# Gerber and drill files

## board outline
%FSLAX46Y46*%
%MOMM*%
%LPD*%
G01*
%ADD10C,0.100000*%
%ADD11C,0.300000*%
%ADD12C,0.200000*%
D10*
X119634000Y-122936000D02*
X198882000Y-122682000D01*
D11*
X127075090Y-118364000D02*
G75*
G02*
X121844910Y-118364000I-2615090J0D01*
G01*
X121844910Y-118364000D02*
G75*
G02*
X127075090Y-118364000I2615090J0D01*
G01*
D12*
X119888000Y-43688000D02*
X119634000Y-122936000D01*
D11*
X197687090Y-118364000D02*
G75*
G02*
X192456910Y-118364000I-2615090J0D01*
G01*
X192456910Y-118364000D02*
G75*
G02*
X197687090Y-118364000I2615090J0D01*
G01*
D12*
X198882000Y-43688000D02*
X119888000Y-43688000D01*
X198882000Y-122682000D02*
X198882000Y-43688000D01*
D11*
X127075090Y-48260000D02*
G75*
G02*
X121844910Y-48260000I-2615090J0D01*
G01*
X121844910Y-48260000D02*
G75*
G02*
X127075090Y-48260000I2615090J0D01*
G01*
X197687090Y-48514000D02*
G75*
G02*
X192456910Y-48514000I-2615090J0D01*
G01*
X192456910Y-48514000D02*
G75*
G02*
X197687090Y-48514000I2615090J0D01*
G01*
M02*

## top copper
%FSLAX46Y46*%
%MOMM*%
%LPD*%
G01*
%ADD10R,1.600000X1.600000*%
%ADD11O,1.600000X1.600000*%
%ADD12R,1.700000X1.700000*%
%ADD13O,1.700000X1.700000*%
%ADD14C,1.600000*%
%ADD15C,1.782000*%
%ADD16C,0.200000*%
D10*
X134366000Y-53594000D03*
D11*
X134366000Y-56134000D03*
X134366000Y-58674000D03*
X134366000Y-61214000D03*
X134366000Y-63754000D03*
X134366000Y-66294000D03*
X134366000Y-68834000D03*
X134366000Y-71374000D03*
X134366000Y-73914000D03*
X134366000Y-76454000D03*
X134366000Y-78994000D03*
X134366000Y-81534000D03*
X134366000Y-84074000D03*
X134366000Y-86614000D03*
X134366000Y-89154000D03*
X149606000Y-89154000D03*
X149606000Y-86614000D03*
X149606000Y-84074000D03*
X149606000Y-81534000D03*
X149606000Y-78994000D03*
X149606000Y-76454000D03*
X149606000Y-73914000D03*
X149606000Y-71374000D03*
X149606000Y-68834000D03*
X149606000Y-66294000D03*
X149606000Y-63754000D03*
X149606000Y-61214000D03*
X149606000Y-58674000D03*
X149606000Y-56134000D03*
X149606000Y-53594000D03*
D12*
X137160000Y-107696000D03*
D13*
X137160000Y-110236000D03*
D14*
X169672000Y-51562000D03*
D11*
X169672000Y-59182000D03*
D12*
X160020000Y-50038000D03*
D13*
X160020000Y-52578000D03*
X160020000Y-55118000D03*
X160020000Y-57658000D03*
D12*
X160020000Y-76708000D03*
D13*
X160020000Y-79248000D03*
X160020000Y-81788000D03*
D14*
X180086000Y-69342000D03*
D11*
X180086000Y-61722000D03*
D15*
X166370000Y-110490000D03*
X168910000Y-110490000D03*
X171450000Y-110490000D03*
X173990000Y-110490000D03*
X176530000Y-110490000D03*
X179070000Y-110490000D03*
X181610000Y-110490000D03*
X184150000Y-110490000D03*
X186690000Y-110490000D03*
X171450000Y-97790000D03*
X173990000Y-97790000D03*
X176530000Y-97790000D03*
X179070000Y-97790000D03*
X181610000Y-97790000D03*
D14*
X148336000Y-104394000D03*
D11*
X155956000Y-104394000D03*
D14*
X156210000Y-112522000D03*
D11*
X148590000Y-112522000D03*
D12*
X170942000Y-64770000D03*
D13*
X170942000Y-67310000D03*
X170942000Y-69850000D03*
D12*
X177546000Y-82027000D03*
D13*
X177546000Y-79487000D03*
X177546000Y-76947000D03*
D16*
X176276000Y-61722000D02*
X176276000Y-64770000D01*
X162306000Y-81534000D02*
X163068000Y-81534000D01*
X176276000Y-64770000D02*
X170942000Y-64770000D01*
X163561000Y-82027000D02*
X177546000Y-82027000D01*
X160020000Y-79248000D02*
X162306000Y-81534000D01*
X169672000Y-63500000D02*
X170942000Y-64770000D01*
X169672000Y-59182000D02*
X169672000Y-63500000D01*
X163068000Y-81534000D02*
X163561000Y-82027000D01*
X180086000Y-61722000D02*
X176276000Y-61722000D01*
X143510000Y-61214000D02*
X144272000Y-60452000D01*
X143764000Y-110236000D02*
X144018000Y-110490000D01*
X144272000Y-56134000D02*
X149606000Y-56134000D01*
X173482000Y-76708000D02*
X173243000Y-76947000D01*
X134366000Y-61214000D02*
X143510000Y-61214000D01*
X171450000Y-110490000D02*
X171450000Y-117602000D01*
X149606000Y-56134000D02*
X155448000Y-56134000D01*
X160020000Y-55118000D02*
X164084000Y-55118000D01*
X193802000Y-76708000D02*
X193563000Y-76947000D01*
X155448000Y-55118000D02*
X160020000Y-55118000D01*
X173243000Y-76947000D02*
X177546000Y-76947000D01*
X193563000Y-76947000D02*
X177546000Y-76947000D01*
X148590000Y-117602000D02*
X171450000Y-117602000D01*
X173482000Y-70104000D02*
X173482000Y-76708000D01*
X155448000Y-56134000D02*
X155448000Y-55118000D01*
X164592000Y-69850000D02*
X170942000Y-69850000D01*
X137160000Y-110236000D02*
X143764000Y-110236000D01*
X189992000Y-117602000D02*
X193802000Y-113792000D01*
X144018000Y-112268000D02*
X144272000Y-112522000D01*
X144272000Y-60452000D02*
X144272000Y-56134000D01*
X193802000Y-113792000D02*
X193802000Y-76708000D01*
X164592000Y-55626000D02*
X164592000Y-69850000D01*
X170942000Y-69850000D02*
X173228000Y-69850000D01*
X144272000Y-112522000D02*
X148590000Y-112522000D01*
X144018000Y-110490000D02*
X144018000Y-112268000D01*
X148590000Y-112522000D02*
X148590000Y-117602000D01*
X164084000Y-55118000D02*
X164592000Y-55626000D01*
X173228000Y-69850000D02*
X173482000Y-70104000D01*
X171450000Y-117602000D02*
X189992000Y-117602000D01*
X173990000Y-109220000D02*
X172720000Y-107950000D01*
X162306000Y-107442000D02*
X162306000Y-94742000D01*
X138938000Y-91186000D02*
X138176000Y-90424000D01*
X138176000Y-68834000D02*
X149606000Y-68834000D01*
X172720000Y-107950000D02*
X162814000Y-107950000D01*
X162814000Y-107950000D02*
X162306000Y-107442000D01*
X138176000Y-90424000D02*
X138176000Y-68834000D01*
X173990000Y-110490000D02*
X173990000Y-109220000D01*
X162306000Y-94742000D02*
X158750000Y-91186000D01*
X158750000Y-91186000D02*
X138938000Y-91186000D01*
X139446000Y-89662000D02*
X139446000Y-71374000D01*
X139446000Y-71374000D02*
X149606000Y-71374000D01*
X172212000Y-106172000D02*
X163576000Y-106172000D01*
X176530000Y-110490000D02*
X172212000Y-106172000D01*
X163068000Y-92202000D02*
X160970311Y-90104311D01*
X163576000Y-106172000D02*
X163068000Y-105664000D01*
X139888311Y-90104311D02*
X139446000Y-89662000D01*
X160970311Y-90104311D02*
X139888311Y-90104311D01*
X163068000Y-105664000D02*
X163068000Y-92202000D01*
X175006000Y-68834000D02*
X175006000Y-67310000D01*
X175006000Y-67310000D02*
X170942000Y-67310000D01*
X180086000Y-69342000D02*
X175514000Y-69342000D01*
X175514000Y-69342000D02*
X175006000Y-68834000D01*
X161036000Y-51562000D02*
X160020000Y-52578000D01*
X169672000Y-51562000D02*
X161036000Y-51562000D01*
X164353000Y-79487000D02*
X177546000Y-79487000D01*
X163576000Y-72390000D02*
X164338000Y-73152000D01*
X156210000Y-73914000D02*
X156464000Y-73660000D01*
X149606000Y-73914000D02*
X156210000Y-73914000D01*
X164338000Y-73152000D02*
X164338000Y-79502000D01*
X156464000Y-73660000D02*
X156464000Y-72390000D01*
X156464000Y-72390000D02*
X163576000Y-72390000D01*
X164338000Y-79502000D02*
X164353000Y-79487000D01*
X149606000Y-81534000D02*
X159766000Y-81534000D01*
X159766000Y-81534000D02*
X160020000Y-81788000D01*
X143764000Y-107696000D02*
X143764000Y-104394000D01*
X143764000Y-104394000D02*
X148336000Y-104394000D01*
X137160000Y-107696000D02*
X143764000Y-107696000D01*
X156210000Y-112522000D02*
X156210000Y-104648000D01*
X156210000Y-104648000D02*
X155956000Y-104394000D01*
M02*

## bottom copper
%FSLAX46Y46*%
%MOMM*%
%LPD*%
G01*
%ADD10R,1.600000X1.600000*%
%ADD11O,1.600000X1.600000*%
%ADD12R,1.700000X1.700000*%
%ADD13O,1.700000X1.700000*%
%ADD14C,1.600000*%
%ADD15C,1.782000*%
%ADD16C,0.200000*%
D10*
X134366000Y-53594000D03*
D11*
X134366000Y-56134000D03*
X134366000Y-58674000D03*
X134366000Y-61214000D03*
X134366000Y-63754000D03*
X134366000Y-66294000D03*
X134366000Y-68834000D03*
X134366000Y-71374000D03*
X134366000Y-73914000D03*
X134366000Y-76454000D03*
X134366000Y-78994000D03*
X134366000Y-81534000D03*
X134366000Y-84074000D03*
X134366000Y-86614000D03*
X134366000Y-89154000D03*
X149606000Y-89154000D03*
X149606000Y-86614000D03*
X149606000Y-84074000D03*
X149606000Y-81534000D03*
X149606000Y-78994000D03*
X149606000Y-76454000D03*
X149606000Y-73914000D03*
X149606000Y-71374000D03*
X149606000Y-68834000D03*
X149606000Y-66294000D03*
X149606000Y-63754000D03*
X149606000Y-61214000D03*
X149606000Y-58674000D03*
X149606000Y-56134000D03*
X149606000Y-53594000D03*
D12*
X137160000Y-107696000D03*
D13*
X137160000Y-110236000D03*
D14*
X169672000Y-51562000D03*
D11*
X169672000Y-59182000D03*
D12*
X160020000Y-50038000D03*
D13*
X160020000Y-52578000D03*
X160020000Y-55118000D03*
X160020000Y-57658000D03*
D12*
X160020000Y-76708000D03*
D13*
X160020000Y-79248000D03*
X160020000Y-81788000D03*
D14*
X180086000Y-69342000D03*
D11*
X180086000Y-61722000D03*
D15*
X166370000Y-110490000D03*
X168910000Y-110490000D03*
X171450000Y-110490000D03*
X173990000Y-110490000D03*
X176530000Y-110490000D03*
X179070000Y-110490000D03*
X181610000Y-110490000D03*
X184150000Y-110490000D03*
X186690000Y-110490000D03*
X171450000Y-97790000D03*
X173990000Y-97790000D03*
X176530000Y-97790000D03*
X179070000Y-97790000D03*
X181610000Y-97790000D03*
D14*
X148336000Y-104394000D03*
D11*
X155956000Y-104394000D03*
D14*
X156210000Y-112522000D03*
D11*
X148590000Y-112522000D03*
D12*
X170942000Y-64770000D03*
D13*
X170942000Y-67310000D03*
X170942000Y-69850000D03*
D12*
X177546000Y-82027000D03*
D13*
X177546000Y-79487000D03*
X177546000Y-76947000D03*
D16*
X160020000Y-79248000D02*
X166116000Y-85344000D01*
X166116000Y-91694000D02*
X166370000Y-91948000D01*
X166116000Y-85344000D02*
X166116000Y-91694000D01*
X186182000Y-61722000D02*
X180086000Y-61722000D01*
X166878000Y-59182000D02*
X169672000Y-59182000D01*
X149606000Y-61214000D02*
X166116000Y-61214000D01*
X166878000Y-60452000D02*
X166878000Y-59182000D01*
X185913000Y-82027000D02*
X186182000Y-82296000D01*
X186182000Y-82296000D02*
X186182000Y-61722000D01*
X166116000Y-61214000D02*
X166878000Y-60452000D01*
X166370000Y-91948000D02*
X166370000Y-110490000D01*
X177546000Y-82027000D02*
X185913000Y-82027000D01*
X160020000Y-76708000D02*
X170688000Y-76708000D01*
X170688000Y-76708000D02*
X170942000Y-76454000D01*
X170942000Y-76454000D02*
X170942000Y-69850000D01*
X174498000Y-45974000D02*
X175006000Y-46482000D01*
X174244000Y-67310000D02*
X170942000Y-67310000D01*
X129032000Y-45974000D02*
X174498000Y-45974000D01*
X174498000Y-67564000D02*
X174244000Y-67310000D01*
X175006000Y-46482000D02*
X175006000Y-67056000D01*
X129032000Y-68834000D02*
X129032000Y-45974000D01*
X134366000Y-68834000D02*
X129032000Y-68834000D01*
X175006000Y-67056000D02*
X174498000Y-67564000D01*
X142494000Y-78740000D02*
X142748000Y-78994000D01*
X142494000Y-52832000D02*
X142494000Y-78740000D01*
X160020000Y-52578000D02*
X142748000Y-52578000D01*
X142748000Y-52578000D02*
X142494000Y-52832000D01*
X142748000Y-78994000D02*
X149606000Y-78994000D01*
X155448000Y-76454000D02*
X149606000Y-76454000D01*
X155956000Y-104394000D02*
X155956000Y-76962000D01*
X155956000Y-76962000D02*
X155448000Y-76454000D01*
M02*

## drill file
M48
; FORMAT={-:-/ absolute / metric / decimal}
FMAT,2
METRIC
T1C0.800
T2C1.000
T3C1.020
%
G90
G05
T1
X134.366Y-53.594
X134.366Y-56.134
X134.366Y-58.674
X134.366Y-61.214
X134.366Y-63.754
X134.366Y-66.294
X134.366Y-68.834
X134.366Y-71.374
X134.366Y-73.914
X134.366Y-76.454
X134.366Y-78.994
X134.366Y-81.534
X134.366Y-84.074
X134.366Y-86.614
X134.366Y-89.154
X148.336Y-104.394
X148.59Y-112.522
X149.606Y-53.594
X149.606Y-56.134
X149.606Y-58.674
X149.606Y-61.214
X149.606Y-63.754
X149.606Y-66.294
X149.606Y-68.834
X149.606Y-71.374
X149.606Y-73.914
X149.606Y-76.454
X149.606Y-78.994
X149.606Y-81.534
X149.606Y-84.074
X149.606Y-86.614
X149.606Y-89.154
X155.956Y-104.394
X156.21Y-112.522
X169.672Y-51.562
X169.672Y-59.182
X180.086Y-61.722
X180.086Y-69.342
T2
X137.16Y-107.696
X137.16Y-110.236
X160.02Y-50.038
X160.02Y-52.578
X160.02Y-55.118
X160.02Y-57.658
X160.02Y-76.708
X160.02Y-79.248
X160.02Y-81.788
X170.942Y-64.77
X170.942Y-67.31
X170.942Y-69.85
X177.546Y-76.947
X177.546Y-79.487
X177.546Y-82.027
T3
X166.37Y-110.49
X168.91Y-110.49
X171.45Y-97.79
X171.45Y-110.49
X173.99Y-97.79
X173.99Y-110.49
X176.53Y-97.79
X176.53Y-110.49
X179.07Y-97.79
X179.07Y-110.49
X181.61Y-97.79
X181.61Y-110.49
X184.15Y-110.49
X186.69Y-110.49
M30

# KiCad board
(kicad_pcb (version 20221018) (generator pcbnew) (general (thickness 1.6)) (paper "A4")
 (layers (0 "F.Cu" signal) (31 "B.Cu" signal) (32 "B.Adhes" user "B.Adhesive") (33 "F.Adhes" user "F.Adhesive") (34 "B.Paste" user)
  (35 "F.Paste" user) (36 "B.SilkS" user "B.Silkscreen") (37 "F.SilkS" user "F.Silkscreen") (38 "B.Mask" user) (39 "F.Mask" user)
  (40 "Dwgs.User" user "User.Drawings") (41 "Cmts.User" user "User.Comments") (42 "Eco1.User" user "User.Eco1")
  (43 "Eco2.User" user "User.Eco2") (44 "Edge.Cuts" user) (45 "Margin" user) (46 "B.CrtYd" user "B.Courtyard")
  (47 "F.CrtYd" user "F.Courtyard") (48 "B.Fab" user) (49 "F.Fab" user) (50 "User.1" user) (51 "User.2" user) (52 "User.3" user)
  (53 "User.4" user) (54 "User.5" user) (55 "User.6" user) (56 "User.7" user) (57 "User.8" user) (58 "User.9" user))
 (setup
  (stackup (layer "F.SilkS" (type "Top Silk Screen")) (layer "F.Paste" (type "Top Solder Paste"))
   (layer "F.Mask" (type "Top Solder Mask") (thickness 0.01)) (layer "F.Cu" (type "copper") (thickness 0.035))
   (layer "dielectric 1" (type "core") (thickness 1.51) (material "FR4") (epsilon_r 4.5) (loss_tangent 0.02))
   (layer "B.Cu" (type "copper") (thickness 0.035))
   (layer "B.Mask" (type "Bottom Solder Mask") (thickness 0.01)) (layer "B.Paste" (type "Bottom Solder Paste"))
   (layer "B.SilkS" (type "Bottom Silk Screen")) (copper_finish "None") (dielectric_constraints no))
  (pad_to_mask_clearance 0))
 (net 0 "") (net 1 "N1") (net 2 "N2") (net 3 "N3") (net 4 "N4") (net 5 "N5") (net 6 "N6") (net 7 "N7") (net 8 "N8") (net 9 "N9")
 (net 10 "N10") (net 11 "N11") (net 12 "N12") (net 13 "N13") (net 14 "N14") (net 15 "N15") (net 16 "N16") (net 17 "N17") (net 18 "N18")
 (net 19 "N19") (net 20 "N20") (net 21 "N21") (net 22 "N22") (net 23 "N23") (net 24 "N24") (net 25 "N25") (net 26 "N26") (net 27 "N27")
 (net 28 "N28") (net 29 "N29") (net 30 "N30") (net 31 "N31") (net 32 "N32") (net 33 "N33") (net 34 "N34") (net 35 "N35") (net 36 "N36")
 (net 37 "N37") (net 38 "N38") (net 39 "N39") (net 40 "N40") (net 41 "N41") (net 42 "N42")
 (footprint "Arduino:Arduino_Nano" (layer "F.Cu") (at 134.366 53.594)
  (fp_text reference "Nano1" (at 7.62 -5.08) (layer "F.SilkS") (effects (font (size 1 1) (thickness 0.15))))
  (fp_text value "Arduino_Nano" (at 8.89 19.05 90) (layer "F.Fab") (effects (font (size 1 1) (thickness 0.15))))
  (pad "1" thru_hole rect (at 0 0) (size 1.6 1.6) (drill 0.8) (layers "*.Cu" "*.Mask") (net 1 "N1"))
  (pad "2" thru_hole oval (at 0 2.54) (size 1.6 1.6) (drill 0.8) (layers "*.Cu" "*.Mask") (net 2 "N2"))
  (pad "3" thru_hole oval (at 0 5.08) (size 1.6 1.6) (drill 0.8) (layers "*.Cu" "*.Mask") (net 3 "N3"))
  (pad "4" thru_hole oval (at 0 7.62) (size 1.6 1.6) (drill 0.8) (layers "*.Cu" "*.Mask") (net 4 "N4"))
  (pad "5" thru_hole oval (at 0 10.16) (size 1.6 1.6) (drill 0.8) (layers "*.Cu" "*.Mask") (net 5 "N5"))
  (pad "6" thru_hole oval (at 0 12.7) (size 1.6 1.6) (drill 0.8) (layers "*.Cu" "*.Mask") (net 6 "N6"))
  (pad "7" thru_hole oval (at 0 15.24) (size 1.6 1.6) (drill 0.8) (layers "*.Cu" "*.Mask") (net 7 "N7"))
  (pad "8" thru_hole oval (at 0 17.78) (size 1.6 1.6) (drill 0.8) (layers "*.Cu" "*.Mask") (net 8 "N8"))
  (pad "9" thru_hole oval (at 0 20.32) (size 1.6 1.6) (drill 0.8) (layers "*.Cu" "*.Mask") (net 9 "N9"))
  (pad "10" thru_hole oval (at 0 22.86) (size 1.6 1.6) (drill 0.8) (layers "*.Cu" "*.Mask") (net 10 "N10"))
  (pad "11" thru_hole oval (at 0 25.4) (size 1.6 1.6) (drill 0.8) (layers "*.Cu" "*.Mask") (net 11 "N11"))
  (pad "12" thru_hole oval (at 0 27.94) (size 1.6 1.6) (drill 0.8) (layers "*.Cu" "*.Mask") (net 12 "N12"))
  (pad "13" thru_hole oval (at 0 30.48) (size 1.6 1.6) (drill 0.8) (layers "*.Cu" "*.Mask") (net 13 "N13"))
  (pad "14" thru_hole oval (at 0 33.02) (size 1.6 1.6) (drill 0.8) (layers "*.Cu" "*.Mask") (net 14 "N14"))
  (pad "15" thru_hole oval (at 0 35.56) (size 1.6 1.6) (drill 0.8) (layers "*.Cu" "*.Mask") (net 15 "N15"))
  (pad "16" thru_hole oval (at 15.24 35.56) (size 1.6 1.6) (drill 0.8) (layers "*.Cu" "*.Mask") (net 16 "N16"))
  (pad "17" thru_hole oval (at 15.24 33.02) (size 1.6 1.6) (drill 0.8) (layers "*.Cu" "*.Mask") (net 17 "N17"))
  (pad "18" thru_hole oval (at 15.24 30.48) (size 1.6 1.6) (drill 0.8) (layers "*.Cu" "*.Mask") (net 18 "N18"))
  (pad "19" thru_hole oval (at 15.24 27.94) (size 1.6 1.6) (drill 0.8) (layers "*.Cu" "*.Mask") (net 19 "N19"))
  (pad "20" thru_hole oval (at 15.24 25.4) (size 1.6 1.6) (drill 0.8) (layers "*.Cu" "*.Mask") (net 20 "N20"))
  (pad "21" thru_hole oval (at 15.24 22.86) (size 1.6 1.6) (drill 0.8) (layers "*.Cu" "*.Mask") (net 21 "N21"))
  (pad "22" thru_hole oval (at 15.24 20.32) (size 1.6 1.6) (drill 0.8) (layers "*.Cu" "*.Mask") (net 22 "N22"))
  (pad "23" thru_hole oval (at 15.24 17.78) (size 1.6 1.6) (drill 0.8) (layers "*.Cu" "*.Mask") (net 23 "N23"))
  (pad "24" thru_hole oval (at 15.24 15.24) (size 1.6 1.6) (drill 0.8) (layers "*.Cu" "*.Mask") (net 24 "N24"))
  (pad "25" thru_hole oval (at 15.24 12.7) (size 1.6 1.6) (drill 0.8) (layers "*.Cu" "*.Mask") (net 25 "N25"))
  (pad "26" thru_hole oval (at 15.24 10.16) (size 1.6 1.6) (drill 0.8) (layers "*.Cu" "*.Mask") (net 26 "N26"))
  (pad "27" thru_hole oval (at 15.24 7.62) (size 1.6 1.6) (drill 0.8) (layers "*.Cu" "*.Mask") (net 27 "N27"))
  (pad "28" thru_hole oval (at 15.24 5.08) (size 1.6 1.6) (drill 0.8) (layers "*.Cu" "*.Mask") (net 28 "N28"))
  (pad "29" thru_hole oval (at 15.24 2.54) (size 1.6 1.6) (drill 0.8) (layers "*.Cu" "*.Mask") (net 4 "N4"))
  (pad "30" thru_hole oval (at 15.24 0) (size 1.6 1.6) (drill 0.8) (layers "*.Cu" "*.Mask") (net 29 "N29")))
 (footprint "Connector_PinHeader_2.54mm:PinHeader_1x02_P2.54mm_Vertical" (layer "F.Cu") (at 137.16 107.696)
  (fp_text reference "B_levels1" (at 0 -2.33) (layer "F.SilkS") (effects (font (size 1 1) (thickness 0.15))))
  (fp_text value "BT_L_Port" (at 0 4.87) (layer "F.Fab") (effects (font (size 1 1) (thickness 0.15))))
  (pad "1" thru_hole rect (at 0 0) (size 1.7 1.7) (drill 1) (layers "*.Cu" "*.Mask") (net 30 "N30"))
  (pad "2" thru_hole oval (at 0 2.54) (size 1.7 1.7) (drill 1) (layers "*.Cu" "*.Mask") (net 4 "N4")))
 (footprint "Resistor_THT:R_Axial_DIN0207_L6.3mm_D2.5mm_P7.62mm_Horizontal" (layer "F.Cu") (at 169.672 51.562 -90)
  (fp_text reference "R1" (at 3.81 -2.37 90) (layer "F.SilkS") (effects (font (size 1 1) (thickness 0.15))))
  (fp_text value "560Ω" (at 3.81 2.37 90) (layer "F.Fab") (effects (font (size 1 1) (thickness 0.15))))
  (pad "1" thru_hole circle (at 0 0 270) (size 1.6 1.6) (drill 0.8) (layers "*.Cu" "*.Mask") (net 20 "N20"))
  (pad "2" thru_hole oval (at 7.62 0 270) (size 1.6 1.6) (drill 0.8) (layers "*.Cu" "*.Mask") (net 27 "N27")))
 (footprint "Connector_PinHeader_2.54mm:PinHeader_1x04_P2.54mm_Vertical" (layer "F.Cu") (at 160.02 50.038)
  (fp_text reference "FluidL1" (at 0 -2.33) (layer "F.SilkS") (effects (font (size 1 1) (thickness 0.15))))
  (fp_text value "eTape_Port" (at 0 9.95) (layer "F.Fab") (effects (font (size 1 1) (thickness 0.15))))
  (pad "1" thru_hole rect (at 0 0) (size 1.7 1.7) (drill 1) (layers "*.Cu" "*.Mask") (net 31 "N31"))
  (pad "2" thru_hole oval (at 0 2.54) (size 1.7 1.7) (drill 1) (layers "*.Cu" "*.Mask") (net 20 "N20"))
  (pad "3" thru_hole oval (at 0 5.08) (size 1.7 1.7) (drill 1) (layers "*.Cu" "*.Mask") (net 4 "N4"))
  (pad "4" thru_hole oval (at 0 7.62) (size 1.7 1.7) (drill 1) (layers "*.Cu" "*.Mask") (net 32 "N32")))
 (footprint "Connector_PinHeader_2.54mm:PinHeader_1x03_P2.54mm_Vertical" (layer "F.Cu") (at 160.02 76.708)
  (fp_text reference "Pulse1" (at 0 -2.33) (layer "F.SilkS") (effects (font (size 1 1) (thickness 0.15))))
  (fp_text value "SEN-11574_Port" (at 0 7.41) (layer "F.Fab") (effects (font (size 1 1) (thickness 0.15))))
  (pad "1" thru_hole rect (at 0 0) (size 1.7 1.7) (drill 1) (layers "*.Cu" "*.Mask") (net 4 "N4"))
  (pad "2" thru_hole oval (at 0 2.54) (size 1.7 1.7) (drill 1) (layers "*.Cu" "*.Mask") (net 27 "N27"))
  (pad "3" thru_hole oval (at 0 5.08) (size 1.7 1.7) (drill 1) (layers "*.Cu" "*.Mask") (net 19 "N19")))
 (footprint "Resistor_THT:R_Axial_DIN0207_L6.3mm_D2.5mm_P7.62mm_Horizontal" (layer "F.Cu") (at 180.086 69.342 90)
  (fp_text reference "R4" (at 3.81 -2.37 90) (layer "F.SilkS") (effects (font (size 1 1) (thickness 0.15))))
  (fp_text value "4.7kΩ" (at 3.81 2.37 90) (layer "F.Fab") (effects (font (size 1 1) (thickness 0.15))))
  (pad "1" thru_hole circle (at 0 0 90) (size 1.6 1.6) (drill 0.8) (layers "*.Cu" "*.Mask") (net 7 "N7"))
  (pad "2" thru_hole oval (at 7.62 0 90) (size 1.6 1.6) (drill 0.8) (layers "*.Cu" "*.Mask") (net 27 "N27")))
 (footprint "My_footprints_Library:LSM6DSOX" (layer "F.Cu") (at 176.53 104.14)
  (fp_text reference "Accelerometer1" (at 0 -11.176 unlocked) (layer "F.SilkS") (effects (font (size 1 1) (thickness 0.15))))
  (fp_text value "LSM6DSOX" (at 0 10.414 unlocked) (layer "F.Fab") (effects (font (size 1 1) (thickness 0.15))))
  (pad "1" thru_hole circle (at -10.16 6.35) (size 1.782 1.782) (drill 1.02) (layers "*.Cu" "*.Mask") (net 27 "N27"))
  (pad "2" thru_hole circle (at -7.62 6.35) (size 1.782 1.782) (drill 1.02) (layers "*.Cu" "*.Mask") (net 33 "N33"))
  (pad "3" thru_hole circle (at -5.08 6.35) (size 1.782 1.782) (drill 1.02) (layers "*.Cu" "*.Mask") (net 4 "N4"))
  (pad "4" thru_hole circle (at -2.54 6.35) (size 1.782 1.782) (drill 1.02) (layers "*.Cu" "*.Mask") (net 24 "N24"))
  (pad "5" thru_hole circle (at 0 6.35) (size 1.782 1.782) (drill 1.02) (layers "*.Cu" "*.Mask") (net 23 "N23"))
  (pad "6" thru_hole circle (at 2.54 6.35) (size 1.782 1.782) (drill 1.02) (layers "*.Cu" "*.Mask") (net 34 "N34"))
  (pad "7" thru_hole circle (at 5.08 6.35) (size 1.782 1.782) (drill 1.02) (layers "*.Cu" "*.Mask") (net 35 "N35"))
  (pad "8" thru_hole circle (at 7.62 6.35) (size 1.782 1.782) (drill 1.02) (layers "*.Cu" "*.Mask") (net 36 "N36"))
  (pad "9" thru_hole circle (at 10.16 6.35) (size 1.782 1.782) (drill 1.02) (layers "*.Cu" "*.Mask") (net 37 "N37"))
  (pad "10" thru_hole circle (at -5.08 -6.35) (size 1.782 1.782) (drill 1.02) (layers "*.Cu" "*.Mask") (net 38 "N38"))
  (pad "11" thru_hole circle (at -2.54 -6.35) (size 1.782 1.782) (drill 1.02) (layers "*.Cu" "*.Mask") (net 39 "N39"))
  (pad "12" thru_hole circle (at 0 -6.35) (size 1.782 1.782) (drill 1.02) (layers "*.Cu" "*.Mask") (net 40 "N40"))
  (pad "13" thru_hole circle (at 2.54 -6.35) (size 1.782 1.782) (drill 1.02) (layers "*.Cu" "*.Mask") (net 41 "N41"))
  (pad "14" thru_hole circle (at 5.08 -6.35) (size 1.782 1.782) (drill 1.02) (layers "*.Cu" "*.Mask") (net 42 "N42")))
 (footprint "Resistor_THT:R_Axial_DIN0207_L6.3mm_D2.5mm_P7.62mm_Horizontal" (layer "F.Cu") (at 148.336 104.394)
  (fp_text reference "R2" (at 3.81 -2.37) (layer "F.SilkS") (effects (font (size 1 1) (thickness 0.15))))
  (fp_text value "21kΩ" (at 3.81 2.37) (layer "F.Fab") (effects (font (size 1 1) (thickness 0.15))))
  (pad "1" thru_hole circle (at 0 0) (size 1.6 1.6) (drill 0.8) (layers "*.Cu" "*.Mask") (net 30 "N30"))
  (pad "2" thru_hole oval (at 7.62 0) (size 1.6 1.6) (drill 0.8) (layers "*.Cu" "*.Mask") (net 21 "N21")))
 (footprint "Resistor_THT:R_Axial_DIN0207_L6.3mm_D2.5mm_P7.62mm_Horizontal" (layer "F.Cu") (at 156.21 112.522 180)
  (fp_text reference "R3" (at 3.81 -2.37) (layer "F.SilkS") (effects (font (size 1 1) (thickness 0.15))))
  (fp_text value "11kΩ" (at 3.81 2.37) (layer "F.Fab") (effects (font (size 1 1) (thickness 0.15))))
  (pad "1" thru_hole circle (at 0 0 180) (size 1.6 1.6) (drill 0.8) (layers "*.Cu" "*.Mask") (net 21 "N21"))
  (pad "2" thru_hole oval (at 7.62 0 180) (size 1.6 1.6) (drill 0.8) (layers "*.Cu" "*.Mask") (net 4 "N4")))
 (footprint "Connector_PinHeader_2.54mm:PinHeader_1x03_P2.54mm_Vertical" (layer "F.Cu") (at 170.942 64.77)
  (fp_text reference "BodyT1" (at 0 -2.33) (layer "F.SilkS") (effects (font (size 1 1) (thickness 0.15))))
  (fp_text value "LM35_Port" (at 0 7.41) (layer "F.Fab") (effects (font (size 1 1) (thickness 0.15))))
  (pad "1" thru_hole rect (at 0 0) (size 1.7 1.7) (drill 1) (layers "*.Cu" "*.Mask") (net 27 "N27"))
  (pad "2" thru_hole oval (at 0 2.54) (size 1.7 1.7) (drill 1) (layers "*.Cu" "*.Mask") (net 7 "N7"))
  (pad "3" thru_hole oval (at 0 5.08) (size 1.7 1.7) (drill 1) (layers "*.Cu" "*.Mask") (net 4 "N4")))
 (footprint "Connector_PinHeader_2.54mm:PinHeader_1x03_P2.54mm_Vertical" (layer "F.Cu") (at 177.546 82.027 180)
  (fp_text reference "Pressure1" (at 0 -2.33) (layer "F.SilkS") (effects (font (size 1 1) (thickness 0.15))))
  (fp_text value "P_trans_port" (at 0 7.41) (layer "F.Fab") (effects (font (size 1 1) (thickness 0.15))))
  (pad "1" thru_hole rect (at 0 0 180) (size 1.7 1.7) (drill 1) (layers "*.Cu" "*.Mask") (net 27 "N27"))
  (pad "2" thru_hole oval (at 0 2.54 180) (size 1.7 1.7) (drill 1) (layers "*.Cu" "*.Mask") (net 22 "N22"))
  (pad "3" thru_hole oval (at 0 5.08 180) (size 1.7 1.7) (drill 1) (layers "*.Cu" "*.Mask") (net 4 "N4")))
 (gr_line (start 119.634 122.936) (end 198.882 122.682) (stroke (width 0.1) (type solid)) (layer "Edge.Cuts"))
 (gr_circle (center 124.46 118.364) (end 127.07509 118.364) (stroke (width 0.3) (type solid)) (fill none) (layer "Edge.Cuts"))
 (gr_line (start 119.888 43.688) (end 119.634 122.936) (stroke (width 0.2) (type solid)) (layer "Edge.Cuts"))
 (gr_circle (center 195.072 118.364) (end 197.68709 118.364) (stroke (width 0.3) (type solid)) (fill none) (layer "Edge.Cuts"))
 (gr_line (start 198.882 43.688) (end 119.888 43.688) (stroke (width 0.2) (type solid)) (layer "Edge.Cuts"))
 (gr_line (start 198.882 122.682) (end 198.882 43.688) (stroke (width 0.2) (type solid)) (layer "Edge.Cuts"))
 (gr_circle (center 124.46 48.26) (end 127.07509 48.26) (stroke (width 0.3) (type solid)) (fill none) (layer "Edge.Cuts"))
 (gr_circle (center 195.072 48.514) (end 197.68709 48.514) (stroke (width 0.3) (type solid)) (fill none) (layer "Edge.Cuts"))
 (segment (start 176.276 61.722) (end 176.276 64.77) (width 0.2) (layer "F.Cu") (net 27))
 (segment (start 162.306 81.534) (end 163.068 81.534) (width 0.2) (layer "F.Cu") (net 27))
 (segment (start 176.276 64.77) (end 170.942 64.77) (width 0.2) (layer "F.Cu") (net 27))
 (segment (start 163.561 82.027) (end 177.546 82.027) (width 0.2) (layer "F.Cu") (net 27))
 (segment (start 160.02 79.248) (end 162.306 81.534) (width 0.2) (layer "F.Cu") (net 27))
 (segment (start 169.672 63.5) (end 170.942 64.77) (width 0.2) (layer "F.Cu") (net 27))
 (segment (start 169.672 59.182) (end 169.672 63.5) (width 0.2) (layer "F.Cu") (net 27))
 (segment (start 163.068 81.534) (end 163.561 82.027) (width 0.2) (layer "F.Cu") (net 27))
 (segment (start 180.086 61.722) (end 176.276 61.722) (width 0.2) (layer "F.Cu") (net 27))
 (segment (start 160.02 79.248) (end 166.116 85.344) (width 0.2) (layer "B.Cu") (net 27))
 (segment (start 166.116 91.694) (end 166.37 91.948) (width 0.2) (layer "B.Cu") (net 27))
 (segment (start 166.116 85.344) (end 166.116 91.694) (width 0.2) (layer "B.Cu") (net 27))
 (segment (start 186.182 61.722) (end 180.086 61.722) (width 0.2) (layer "B.Cu") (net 27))
 (segment (start 166.878 59.182) (end 169.672 59.182) (width 0.2) (layer "B.Cu") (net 27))
 (segment (start 149.606 61.214) (end 166.116 61.214) (width 0.2) (layer "B.Cu") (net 27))
 (segment (start 166.878 60.452) (end 166.878 59.182) (width 0.2) (layer "B.Cu") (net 27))
 (segment (start 185.913 82.027) (end 186.182 82.296) (width 0.2) (layer "B.Cu") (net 27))
 (segment (start 186.182 82.296) (end 186.182 61.722) (width 0.2) (layer "B.Cu") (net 27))
 (segment (start 166.116 61.214) (end 166.878 60.452) (width 0.2) (layer "B.Cu") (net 27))
 (segment (start 166.37 91.948) (end 166.37 110.49) (width 0.2) (layer "B.Cu") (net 27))
 (segment (start 177.546 82.027) (end 185.913 82.027) (width 0.2) (layer "B.Cu") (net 27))
 (segment (start 143.51 61.214) (end 144.272 60.452) (width 0.2) (layer "F.Cu") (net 4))
 (segment (start 143.764 110.236) (end 144.018 110.49) (width 0.2) (layer "F.Cu") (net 4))
 (segment (start 144.272 56.134) (end 149.606 56.134) (width 0.2) (layer "F.Cu") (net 4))
 (segment (start 173.482 76.708) (end 173.243 76.947) (width 0.2) (layer "F.Cu") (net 4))
 (segment (start 134.366 61.214) (end 143.51 61.214) (width 0.2) (layer "F.Cu") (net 4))
 (segment (start 171.45 110.49) (end 171.45 117.602) (width 0.2) (layer "F.Cu") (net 4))
 (segment (start 149.606 56.134) (end 155.448 56.134) (width 0.2) (layer "F.Cu") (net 4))
 (segment (start 160.02 55.118) (end 164.084 55.118) (width 0.2) (layer "F.Cu") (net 4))
 (segment (start 193.802 76.708) (end 193.563 76.947) (width 0.2) (layer "F.Cu") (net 4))
 (segment (start 155.448 55.118) (end 160.02 55.118) (width 0.2) (layer "F.Cu") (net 4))
 (segment (start 173.243 76.947) (end 177.546 76.947) (width 0.2) (layer "F.Cu") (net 4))
 (segment (start 193.563 76.947) (end 177.546 76.947) (width 0.2) (layer "F.Cu") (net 4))
 (segment (start 148.59 117.602) (end 171.45 117.602) (width 0.2) (layer "F.Cu") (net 4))
 (segment (start 173.482 70.104) (end 173.482 76.708) (width 0.2) (layer "F.Cu") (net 4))
 (segment (start 155.448 56.134) (end 155.448 55.118) (width 0.2) (layer "F.Cu") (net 4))
 (segment (start 164.592 69.85) (end 170.942 69.85) (width 0.2) (layer "F.Cu") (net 4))
 (segment (start 137.16 110.236) (end 143.764 110.236) (width 0.2) (layer "F.Cu") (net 4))
 (segment (start 189.992 117.602) (end 193.802 113.792) (width 0.2) (layer "F.Cu") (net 4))
 (segment (start 144.018 112.268) (end 144.272 112.522) (width 0.2) (layer "F.Cu") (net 4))
 (segment (start 144.272 60.452) (end 144.272 56.134) (width 0.2) (layer "F.Cu") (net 4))
 (segment (start 193.802 113.792) (end 193.802 76.708) (width 0.2) (layer "F.Cu") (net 4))
 (segment (start 164.592 55.626) (end 164.592 69.85) (width 0.2) (layer "F.Cu") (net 4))
 (segment (start 170.942 69.85) (end 173.228 69.85) (width 0.2) (layer "F.Cu") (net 4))
 (segment (start 144.272 112.522) (end 148.59 112.522) (width 0.2) (layer "F.Cu") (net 4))
 (segment (start 144.018 110.49) (end 144.018 112.268) (width 0.2) (layer "F.Cu") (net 4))
 (segment (start 148.59 112.522) (end 148.59 117.602) (width 0.2) (layer "F.Cu") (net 4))
 (segment (start 164.084 55.118) (end 164.592 55.626) (width 0.2) (layer "F.Cu") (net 4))
 (segment (start 173.228 69.85) (end 173.482 70.104) (width 0.2) (layer "F.Cu") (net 4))
 (segment (start 171.45 117.602) (end 189.992 117.602) (width 0.2) (layer "F.Cu") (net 4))
 (segment (start 160.02 76.708) (end 170.688 76.708) (width 0.2) (layer "B.Cu") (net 4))
 (segment (start 170.688 76.708) (end 170.942 76.454) (width 0.2) (layer "B.Cu") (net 4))
 (segment (start 170.942 76.454) (end 170.942 69.85) (width 0.2) (layer "B.Cu") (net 4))
 (segment (start 173.99 109.22) (end 172.72 107.95) (width 0.2) (layer "F.Cu") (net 24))
 (segment (start 162.306 107.442) (end 162.306 94.742) (width 0.2) (layer "F.Cu") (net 24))
 (segment (start 138.938 91.186) (end 138.176 90.424) (width 0.2) (layer "F.Cu") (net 24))
 (segment (start 138.176 68.834) (end 149.606 68.834) (width 0.2) (layer "F.Cu") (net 24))
 (segment (start 172.72 107.95) (end 162.814 107.95) (width 0.2) (layer "F.Cu") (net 24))
 (segment (start 162.814 107.95) (end 162.306 107.442) (width 0.2) (layer "F.Cu") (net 24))
 (segment (start 138.176 90.424) (end 138.176 68.834) (width 0.2) (layer "F.Cu") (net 24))
 (segment (start 173.99 110.49) (end 173.99 109.22) (width 0.2) (layer "F.Cu") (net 24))
 (segment (start 162.306 94.742) (end 158.75 91.186) (width 0.2) (layer "F.Cu") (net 24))
 (segment (start 158.75 91.186) (end 138.938 91.186) (width 0.2) (layer "F.Cu") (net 24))
 (segment (start 139.446 89.662) (end 139.446 71.374) (width 0.2) (layer "F.Cu") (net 23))
 (segment (start 139.446 71.374) (end 149.606 71.374) (width 0.2) (layer "F.Cu") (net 23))
 (segment (start 172.212 106.172) (end 163.576 106.172) (width 0.2) (layer "F.Cu") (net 23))
 (segment (start 176.53 110.49) (end 172.212 106.172) (width 0.2) (layer "F.Cu") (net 23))
 (segment (start 163.068 92.202) (end 160.970311 90.104311) (width 0.2) (layer "F.Cu") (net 23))
 (segment (start 163.576 106.172) (end 163.068 105.664) (width 0.2) (layer "F.Cu") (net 23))
 (segment (start 139.888311 90.104311) (end 139.446 89.662) (width 0.2) (layer "F.Cu") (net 23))
 (segment (start 160.970311 90.104311) (end 139.888311 90.104311) (width 0.2) (layer "F.Cu") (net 23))
 (segment (start 163.068 105.664) (end 163.068 92.202) (width 0.2) (layer "F.Cu") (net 23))
 (segment (start 175.006 68.834) (end 175.006 67.31) (width 0.2) (layer "F.Cu") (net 7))
 (segment (start 175.006 67.31) (end 170.942 67.31) (width 0.2) (layer "F.Cu") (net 7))
 (segment (start 180.086 69.342) (end 175.514 69.342) (width 0.2) (layer "F.Cu") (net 7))
 (segment (start 175.514 69.342) (end 175.006 68.834) (width 0.2) (layer "F.Cu") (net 7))
 (segment (start 174.498 45.974) (end 175.006 46.482) (width 0.2) (layer "B.Cu") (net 7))
 (segment (start 174.244 67.31) (end 170.942 67.31) (width 0.2) (layer "B.Cu") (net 7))
 (segment (start 129.032 45.974) (end 174.498 45.974) (width 0.2) (layer "B.Cu") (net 7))
 (segment (start 174.498 67.564) (end 174.244 67.31) (width 0.2) (layer "B.Cu") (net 7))
 (segment (start 175.006 46.482) (end 175.006 67.056) (width 0.2) (layer "B.Cu") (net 7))
 (segment (start 129.032 68.834) (end 129.032 45.974) (width 0.2) (layer "B.Cu") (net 7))
 (segment (start 134.366 68.834) (end 129.032 68.834) (width 0.2) (layer "B.Cu") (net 7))
 (segment (start 175.006 67.056) (end 174.498 67.564) (width 0.2) (layer "B.Cu") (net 7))
 (segment (start 161.036 51.562) (end 160.02 52.578) (width 0.2) (layer "F.Cu") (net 20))
 (segment (start 169.672 51.562) (end 161.036 51.562) (width 0.2) (layer "F.Cu") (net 20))
 (segment (start 142.494 78.74) (end 142.748 78.994) (width 0.2) (layer "B.Cu") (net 20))
 (segment (start 142.494 52.832) (end 142.494 78.74) (width 0.2) (layer "B.Cu") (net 20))
 (segment (start 160.02 52.578) (end 142.748 52.578) (width 0.2) (layer "B.Cu") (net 20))
 (segment (start 142.748 52.578) (end 142.494 52.832) (width 0.2) (layer "B.Cu") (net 20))
 (segment (start 142.748 78.994) (end 149.606 78.994) (width 0.2) (layer "B.Cu") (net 20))
 (segment (start 164.353 79.487) (end 177.546 79.487) (width 0.2) (layer "F.Cu") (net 22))
 (segment (start 163.576 72.39) (end 164.338 73.152) (width 0.2) (layer "F.Cu") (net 22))
 (segment (start 156.21 73.914) (end 156.464 73.66) (width 0.2) (layer "F.Cu") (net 22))
 (segment (start 149.606 73.914) (end 156.21 73.914) (width 0.2) (layer "F.Cu") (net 22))
 (segment (start 164.338 73.152) (end 164.338 79.502) (width 0.2) (layer "F.Cu") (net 22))
 (segment (start 156.464 73.66) (end 156.464 72.39) (width 0.2) (layer "F.Cu") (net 22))
 (segment (start 156.464 72.39) (end 163.576 72.39) (width 0.2) (layer "F.Cu") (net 22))
 (segment (start 164.338 79.502) (end 164.353 79.487) (width 0.2) (layer "F.Cu") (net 22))
 (segment (start 149.606 81.534) (end 159.766 81.534) (width 0.2) (layer "F.Cu") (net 19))
 (segment (start 159.766 81.534) (end 160.02 81.788) (width 0.2) (layer "F.Cu") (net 19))
 (segment (start 143.764 107.696) (end 143.764 104.394) (width 0.2) (layer "F.Cu") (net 30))
 (segment (start 143.764 104.394) (end 148.336 104.394) (width 0.2) (layer "F.Cu") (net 30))
 (segment (start 137.16 107.696) (end 143.764 107.696) (width 0.2) (layer "F.Cu") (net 30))
 (segment (start 156.21 112.522) (end 156.21 104.648) (width 0.2) (layer "F.Cu") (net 21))
 (segment (start 156.21 104.648) (end 155.956 104.394) (width 0.2) (layer "F.Cu") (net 21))
 (segment (start 155.448 76.454) (end 149.606 76.454) (width 0.2) (layer "B.Cu") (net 21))
 (segment (start 155.956 104.394) (end 155.956 76.962) (width 0.2) (layer "B.Cu") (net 21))
 (segment (start 155.956 76.962) (end 155.448 76.454) (width 0.2) (layer "B.Cu") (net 21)))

